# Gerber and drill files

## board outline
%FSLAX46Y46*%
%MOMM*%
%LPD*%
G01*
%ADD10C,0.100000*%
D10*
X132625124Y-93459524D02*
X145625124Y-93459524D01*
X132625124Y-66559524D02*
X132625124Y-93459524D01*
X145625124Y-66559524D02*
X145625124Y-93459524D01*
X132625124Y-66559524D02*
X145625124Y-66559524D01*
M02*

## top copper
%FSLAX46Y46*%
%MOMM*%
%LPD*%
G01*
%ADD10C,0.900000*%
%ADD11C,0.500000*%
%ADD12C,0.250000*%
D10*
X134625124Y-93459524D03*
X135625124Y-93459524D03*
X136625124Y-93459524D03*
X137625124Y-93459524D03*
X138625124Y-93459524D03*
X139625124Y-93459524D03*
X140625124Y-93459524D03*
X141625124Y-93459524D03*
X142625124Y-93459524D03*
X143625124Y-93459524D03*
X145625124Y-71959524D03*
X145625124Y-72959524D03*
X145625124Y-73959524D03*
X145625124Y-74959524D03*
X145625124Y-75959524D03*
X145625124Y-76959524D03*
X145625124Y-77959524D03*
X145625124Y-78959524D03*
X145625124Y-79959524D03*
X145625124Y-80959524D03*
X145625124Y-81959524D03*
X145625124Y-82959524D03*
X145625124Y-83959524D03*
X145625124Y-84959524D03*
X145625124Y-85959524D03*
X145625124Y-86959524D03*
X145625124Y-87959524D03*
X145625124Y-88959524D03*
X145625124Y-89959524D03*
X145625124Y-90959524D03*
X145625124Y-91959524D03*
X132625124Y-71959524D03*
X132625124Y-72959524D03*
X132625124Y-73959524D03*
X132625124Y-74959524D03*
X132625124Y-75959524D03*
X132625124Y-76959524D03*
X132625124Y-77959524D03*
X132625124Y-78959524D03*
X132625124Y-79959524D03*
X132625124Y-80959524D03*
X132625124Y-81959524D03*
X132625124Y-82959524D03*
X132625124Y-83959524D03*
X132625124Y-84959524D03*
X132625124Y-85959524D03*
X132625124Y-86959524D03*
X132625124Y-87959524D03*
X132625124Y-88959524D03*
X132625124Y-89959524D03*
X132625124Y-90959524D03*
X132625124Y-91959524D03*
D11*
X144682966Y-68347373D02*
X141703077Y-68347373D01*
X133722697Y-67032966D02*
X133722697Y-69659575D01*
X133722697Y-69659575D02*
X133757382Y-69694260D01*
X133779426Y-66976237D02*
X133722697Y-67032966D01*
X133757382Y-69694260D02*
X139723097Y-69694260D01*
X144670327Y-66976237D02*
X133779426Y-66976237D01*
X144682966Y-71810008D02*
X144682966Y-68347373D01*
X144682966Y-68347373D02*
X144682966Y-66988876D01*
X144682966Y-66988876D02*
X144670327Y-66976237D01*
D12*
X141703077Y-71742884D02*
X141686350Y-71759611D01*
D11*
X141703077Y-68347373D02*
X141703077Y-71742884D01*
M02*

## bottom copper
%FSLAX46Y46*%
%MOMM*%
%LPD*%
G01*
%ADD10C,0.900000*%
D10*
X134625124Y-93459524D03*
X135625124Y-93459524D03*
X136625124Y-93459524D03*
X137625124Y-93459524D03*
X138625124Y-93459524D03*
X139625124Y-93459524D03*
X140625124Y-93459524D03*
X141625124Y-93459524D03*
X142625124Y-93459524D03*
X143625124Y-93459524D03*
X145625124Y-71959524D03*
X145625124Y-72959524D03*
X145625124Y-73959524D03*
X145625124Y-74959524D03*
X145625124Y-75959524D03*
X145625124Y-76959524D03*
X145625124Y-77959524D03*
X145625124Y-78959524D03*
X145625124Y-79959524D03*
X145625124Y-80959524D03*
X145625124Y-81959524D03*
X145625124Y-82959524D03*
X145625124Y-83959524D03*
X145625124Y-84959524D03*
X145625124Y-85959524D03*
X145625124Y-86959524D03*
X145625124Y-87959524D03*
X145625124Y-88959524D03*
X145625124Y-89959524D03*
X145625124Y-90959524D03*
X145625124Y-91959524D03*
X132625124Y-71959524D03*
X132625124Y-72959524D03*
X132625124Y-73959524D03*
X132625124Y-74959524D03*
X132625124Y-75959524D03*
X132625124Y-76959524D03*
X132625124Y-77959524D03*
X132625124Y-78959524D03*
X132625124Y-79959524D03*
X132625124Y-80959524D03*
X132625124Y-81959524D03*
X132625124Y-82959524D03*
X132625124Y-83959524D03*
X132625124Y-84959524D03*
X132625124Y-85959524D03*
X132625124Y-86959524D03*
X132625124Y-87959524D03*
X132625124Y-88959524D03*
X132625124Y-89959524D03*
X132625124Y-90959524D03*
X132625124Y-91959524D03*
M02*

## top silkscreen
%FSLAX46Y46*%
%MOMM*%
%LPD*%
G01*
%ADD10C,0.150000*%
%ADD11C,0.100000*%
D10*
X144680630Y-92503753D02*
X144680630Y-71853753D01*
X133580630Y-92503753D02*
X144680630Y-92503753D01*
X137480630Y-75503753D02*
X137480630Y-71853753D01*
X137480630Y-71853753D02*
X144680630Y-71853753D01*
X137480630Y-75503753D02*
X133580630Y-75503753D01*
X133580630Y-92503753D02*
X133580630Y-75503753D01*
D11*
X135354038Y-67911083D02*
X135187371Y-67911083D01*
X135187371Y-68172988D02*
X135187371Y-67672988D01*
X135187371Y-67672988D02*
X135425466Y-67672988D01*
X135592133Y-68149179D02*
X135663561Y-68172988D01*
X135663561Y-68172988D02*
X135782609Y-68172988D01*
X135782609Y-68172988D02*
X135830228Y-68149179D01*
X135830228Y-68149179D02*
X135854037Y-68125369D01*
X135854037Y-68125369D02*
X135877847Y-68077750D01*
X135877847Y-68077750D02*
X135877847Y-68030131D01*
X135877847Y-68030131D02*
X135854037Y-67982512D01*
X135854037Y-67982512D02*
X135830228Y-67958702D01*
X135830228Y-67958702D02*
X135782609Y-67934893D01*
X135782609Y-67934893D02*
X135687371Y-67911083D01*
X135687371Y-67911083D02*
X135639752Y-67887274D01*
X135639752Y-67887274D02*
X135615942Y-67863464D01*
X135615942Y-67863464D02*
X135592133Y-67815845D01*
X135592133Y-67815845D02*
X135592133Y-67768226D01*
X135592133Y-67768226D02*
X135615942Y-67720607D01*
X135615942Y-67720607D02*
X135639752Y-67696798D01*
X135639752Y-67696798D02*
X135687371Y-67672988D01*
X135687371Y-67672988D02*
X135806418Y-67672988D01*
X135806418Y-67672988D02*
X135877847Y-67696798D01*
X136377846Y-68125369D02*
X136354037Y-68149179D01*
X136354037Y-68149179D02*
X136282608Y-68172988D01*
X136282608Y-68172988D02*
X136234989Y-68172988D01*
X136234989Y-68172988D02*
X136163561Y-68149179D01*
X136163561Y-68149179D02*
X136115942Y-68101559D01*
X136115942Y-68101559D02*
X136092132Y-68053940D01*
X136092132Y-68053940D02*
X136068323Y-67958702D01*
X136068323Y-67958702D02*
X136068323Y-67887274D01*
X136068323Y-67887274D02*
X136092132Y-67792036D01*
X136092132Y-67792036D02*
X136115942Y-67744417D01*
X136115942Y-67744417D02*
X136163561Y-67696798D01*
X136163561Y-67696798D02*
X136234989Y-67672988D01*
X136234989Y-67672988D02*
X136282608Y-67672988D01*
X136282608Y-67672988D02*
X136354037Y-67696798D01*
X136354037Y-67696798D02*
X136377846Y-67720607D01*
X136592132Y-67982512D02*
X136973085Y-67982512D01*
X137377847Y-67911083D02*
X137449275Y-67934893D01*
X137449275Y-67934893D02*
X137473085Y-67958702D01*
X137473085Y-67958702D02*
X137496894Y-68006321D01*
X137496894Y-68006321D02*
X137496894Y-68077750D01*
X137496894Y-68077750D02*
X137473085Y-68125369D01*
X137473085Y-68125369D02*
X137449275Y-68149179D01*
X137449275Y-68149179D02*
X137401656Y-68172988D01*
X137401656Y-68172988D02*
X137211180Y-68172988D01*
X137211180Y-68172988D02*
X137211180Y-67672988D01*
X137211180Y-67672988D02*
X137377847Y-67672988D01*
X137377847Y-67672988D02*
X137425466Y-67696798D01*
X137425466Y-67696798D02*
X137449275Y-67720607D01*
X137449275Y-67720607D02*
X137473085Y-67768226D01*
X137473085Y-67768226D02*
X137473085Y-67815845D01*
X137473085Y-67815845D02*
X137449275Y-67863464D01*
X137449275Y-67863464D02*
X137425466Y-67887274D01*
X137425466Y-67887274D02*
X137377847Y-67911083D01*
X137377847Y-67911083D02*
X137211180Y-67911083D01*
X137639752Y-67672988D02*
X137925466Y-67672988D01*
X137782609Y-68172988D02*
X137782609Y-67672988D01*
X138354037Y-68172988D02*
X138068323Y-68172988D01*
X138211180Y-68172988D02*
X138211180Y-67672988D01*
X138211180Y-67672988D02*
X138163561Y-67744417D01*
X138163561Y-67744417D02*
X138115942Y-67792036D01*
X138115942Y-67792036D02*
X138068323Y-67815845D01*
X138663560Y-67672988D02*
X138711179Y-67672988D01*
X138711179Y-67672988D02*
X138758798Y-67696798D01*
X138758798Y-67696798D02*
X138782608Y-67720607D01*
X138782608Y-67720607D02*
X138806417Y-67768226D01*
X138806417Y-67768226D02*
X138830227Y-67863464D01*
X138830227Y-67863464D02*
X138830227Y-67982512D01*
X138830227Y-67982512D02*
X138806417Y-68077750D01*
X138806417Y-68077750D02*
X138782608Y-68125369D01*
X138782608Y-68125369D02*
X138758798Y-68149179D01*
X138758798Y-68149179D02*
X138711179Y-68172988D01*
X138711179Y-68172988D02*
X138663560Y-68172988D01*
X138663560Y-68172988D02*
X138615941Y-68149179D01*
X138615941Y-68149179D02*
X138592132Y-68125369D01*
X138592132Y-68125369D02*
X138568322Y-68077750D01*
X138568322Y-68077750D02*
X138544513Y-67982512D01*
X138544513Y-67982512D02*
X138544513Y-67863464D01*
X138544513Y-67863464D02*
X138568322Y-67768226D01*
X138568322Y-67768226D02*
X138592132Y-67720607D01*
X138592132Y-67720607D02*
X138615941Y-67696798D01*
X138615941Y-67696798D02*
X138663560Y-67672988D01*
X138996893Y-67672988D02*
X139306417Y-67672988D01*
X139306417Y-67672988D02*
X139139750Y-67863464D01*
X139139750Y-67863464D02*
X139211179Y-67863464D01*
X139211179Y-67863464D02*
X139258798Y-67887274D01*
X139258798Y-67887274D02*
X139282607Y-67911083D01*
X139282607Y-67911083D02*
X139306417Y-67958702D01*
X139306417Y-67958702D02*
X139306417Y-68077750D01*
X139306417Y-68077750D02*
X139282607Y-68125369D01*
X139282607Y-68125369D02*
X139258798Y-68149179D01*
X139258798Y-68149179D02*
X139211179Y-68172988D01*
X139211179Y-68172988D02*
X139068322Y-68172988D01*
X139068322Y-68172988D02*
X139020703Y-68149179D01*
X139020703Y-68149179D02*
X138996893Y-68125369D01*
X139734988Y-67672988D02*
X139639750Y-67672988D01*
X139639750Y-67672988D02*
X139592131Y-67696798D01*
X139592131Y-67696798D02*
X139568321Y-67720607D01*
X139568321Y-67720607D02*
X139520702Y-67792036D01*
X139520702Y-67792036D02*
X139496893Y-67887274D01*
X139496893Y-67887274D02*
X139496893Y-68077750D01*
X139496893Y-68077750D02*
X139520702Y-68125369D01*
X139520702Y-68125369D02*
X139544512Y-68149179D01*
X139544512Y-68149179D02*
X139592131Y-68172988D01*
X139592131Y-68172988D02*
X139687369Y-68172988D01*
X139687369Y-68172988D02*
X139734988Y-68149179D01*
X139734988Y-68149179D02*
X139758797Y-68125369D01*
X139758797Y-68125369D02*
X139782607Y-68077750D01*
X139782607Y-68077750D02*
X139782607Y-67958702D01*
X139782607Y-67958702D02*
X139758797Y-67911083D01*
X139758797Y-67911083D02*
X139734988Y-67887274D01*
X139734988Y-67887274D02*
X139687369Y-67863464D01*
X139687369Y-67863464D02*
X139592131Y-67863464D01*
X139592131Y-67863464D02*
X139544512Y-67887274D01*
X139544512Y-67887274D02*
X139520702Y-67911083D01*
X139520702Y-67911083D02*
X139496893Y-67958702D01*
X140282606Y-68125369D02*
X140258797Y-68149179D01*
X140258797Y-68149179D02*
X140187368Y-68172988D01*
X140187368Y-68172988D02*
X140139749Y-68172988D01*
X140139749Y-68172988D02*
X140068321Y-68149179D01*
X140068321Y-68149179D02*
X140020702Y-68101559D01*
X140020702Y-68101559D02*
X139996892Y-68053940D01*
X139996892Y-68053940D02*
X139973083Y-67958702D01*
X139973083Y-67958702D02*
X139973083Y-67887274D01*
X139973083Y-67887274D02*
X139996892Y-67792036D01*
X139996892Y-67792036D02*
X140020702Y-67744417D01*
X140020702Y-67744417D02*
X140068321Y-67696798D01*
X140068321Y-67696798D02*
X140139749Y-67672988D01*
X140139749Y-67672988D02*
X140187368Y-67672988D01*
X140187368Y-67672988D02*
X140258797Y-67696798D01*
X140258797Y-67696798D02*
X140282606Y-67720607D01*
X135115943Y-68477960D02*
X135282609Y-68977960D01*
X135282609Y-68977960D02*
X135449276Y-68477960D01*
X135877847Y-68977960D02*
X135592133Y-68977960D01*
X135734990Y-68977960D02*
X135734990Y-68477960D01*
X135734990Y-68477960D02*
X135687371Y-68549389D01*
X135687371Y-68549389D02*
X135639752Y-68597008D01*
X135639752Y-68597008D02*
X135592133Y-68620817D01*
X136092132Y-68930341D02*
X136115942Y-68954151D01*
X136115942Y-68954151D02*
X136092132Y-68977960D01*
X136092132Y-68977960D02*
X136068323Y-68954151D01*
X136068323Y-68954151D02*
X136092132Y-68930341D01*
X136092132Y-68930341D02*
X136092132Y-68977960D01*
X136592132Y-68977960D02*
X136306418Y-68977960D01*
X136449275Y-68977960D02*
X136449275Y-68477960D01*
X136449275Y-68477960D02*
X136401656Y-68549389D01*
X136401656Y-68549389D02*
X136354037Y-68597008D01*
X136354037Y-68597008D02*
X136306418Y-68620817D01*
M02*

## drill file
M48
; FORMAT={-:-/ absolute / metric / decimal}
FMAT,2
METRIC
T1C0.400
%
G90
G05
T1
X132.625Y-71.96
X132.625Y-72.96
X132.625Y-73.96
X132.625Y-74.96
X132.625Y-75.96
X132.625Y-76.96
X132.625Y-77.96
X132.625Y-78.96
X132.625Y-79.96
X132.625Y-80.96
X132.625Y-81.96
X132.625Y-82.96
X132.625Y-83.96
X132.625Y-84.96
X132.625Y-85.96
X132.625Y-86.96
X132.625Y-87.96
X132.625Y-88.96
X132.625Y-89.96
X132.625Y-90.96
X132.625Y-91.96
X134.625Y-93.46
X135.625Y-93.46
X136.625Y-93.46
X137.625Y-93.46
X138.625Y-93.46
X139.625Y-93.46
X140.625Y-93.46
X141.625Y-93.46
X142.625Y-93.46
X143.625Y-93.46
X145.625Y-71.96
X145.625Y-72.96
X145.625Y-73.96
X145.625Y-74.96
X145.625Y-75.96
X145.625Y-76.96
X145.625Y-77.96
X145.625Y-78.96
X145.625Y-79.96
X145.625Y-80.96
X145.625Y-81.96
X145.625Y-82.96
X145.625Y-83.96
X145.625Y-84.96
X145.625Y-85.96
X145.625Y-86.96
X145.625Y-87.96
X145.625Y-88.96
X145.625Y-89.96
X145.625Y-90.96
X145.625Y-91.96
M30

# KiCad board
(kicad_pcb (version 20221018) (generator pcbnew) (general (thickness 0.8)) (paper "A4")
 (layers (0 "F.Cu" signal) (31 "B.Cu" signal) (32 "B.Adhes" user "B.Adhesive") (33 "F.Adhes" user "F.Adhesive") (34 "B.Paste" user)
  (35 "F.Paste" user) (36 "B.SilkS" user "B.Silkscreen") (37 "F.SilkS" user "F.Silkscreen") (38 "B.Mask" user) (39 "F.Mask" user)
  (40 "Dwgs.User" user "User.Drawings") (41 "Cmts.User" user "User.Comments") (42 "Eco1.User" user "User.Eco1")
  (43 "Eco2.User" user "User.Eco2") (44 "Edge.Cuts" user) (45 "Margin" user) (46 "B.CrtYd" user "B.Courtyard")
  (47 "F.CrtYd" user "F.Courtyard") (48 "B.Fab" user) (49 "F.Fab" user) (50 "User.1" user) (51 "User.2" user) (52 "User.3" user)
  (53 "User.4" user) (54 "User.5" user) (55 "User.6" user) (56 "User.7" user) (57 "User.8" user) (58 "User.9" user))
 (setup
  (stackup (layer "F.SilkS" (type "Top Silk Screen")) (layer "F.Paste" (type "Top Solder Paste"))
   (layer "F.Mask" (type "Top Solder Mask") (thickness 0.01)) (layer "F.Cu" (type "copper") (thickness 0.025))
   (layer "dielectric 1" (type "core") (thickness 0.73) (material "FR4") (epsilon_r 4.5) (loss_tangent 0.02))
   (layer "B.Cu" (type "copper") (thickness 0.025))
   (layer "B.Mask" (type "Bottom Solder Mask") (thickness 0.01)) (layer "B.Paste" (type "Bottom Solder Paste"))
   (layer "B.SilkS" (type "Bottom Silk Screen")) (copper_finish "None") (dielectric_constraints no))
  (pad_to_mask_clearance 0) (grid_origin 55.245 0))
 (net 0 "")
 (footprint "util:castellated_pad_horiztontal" (layer "F.Cu") (at 134.625124 93.459524)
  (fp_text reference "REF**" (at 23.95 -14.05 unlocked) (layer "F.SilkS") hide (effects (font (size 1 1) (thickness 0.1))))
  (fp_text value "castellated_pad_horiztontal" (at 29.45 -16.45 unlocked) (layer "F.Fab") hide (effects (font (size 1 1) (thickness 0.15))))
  (pad "1" thru_hole circle (at 0 0) (size 0.9 0.9) (drill 0.4) (layers "*.Cu" "*.Mask"))
  (pad "1" thru_hole circle (at 1 0) (size 0.9 0.9) (drill 0.4) (layers "*.Cu" "*.Mask"))
  (pad "1" thru_hole circle (at 2 0) (size 0.9 0.9) (drill 0.4) (layers "*.Cu" "*.Mask"))
  (pad "1" thru_hole circle (at 3 0) (size 0.9 0.9) (drill 0.4) (layers "*.Cu" "*.Mask"))
  (pad "1" thru_hole circle (at 4 0) (size 0.9 0.9) (drill 0.4) (layers "*.Cu" "*.Mask"))
  (pad "1" thru_hole circle (at 5 0) (size 0.9 0.9) (drill 0.4) (layers "*.Cu" "*.Mask"))
  (pad "1" thru_hole circle (at 6 0) (size 0.9 0.9) (drill 0.4) (layers "*.Cu" "*.Mask"))
  (pad "1" thru_hole circle (at 7 0) (size 0.9 0.9) (drill 0.4) (layers "*.Cu" "*.Mask"))
  (pad "1" thru_hole circle (at 8 0) (size 0.9 0.9) (drill 0.4) (layers "*.Cu" "*.Mask"))
  (pad "1" thru_hole circle (at 9 0) (size 0.9 0.9) (drill 0.4) (layers "*.Cu" "*.Mask")))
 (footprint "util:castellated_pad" (layer "F.Cu") (at 145.625124 71.959524)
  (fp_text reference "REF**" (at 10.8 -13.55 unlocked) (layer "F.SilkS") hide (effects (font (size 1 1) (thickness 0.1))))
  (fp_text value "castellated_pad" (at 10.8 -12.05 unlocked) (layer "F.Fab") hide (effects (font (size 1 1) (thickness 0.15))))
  (pad "1" thru_hole circle (at 0 0) (size 0.9 0.9) (drill 0.4) (layers "*.Cu" "*.Mask"))
  (pad "1" thru_hole circle (at 0 1) (size 0.9 0.9) (drill 0.4) (layers "*.Cu" "*.Mask"))
  (pad "1" thru_hole circle (at 0 2) (size 0.9 0.9) (drill 0.4) (layers "*.Cu" "*.Mask"))
  (pad "1" thru_hole circle (at 0 3) (size 0.9 0.9) (drill 0.4) (layers "*.Cu" "*.Mask"))
  (pad "1" thru_hole circle (at 0 4) (size 0.9 0.9) (drill 0.4) (layers "*.Cu" "*.Mask"))
  (pad "1" thru_hole circle (at 0 5) (size 0.9 0.9) (drill 0.4) (layers "*.Cu" "*.Mask"))
  (pad "1" thru_hole circle (at 0 6) (size 0.9 0.9) (drill 0.4) (layers "*.Cu" "*.Mask"))
  (pad "1" thru_hole circle (at 0 7) (size 0.9 0.9) (drill 0.4) (layers "*.Cu" "*.Mask"))
  (pad "1" thru_hole circle (at 0 8) (size 0.9 0.9) (drill 0.4) (layers "*.Cu" "*.Mask"))
  (pad "1" thru_hole circle (at 0 9) (size 0.9 0.9) (drill 0.4) (layers "*.Cu" "*.Mask"))
  (pad "1" thru_hole circle (at 0 10) (size 0.9 0.9) (drill 0.4) (layers "*.Cu" "*.Mask"))
  (pad "1" thru_hole circle (at 0 11) (size 0.9 0.9) (drill 0.4) (layers "*.Cu" "*.Mask"))
  (pad "1" thru_hole circle (at 0 12) (size 0.9 0.9) (drill 0.4) (layers "*.Cu" "*.Mask"))
  (pad "1" thru_hole circle (at 0 13) (size 0.9 0.9) (drill 0.4) (layers "*.Cu" "*.Mask"))
  (pad "1" thru_hole circle (at 0 14) (size 0.9 0.9) (drill 0.4) (layers "*.Cu" "*.Mask"))
  (pad "1" thru_hole circle (at 0 15) (size 0.9 0.9) (drill 0.4) (layers "*.Cu" "*.Mask"))
  (pad "1" thru_hole circle (at 0 16) (size 0.9 0.9) (drill 0.4) (layers "*.Cu" "*.Mask"))
  (pad "1" thru_hole circle (at 0 17) (size 0.9 0.9) (drill 0.4) (layers "*.Cu" "*.Mask"))
  (pad "1" thru_hole circle (at 0 18) (size 0.9 0.9) (drill 0.4) (layers "*.Cu" "*.Mask"))
  (pad "1" thru_hole circle (at 0 19) (size 0.9 0.9) (drill 0.4) (layers "*.Cu" "*.Mask"))
  (pad "1" thru_hole circle (at 0 20) (size 0.9 0.9) (drill 0.4) (layers "*.Cu" "*.Mask")))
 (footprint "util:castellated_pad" (layer "F.Cu") (at 132.625124 71.959524)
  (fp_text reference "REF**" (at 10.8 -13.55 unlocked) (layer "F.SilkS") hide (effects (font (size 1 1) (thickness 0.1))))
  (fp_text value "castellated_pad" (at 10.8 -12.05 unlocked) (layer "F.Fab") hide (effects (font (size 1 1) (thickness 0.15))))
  (pad "1" thru_hole circle (at 0 0) (size 0.9 0.9) (drill 0.4) (layers "*.Cu" "*.Mask"))
  (pad "1" thru_hole circle (at 0 1) (size 0.9 0.9) (drill 0.4) (layers "*.Cu" "*.Mask"))
  (pad "1" thru_hole circle (at 0 2) (size 0.9 0.9) (drill 0.4) (layers "*.Cu" "*.Mask"))
  (pad "1" thru_hole circle (at 0 3) (size 0.9 0.9) (drill 0.4) (layers "*.Cu" "*.Mask"))
  (pad "1" thru_hole circle (at 0 4) (size 0.9 0.9) (drill 0.4) (layers "*.Cu" "*.Mask"))
  (pad "1" thru_hole circle (at 0 5) (size 0.9 0.9) (drill 0.4) (layers "*.Cu" "*.Mask"))
  (pad "1" thru_hole circle (at 0 6) (size 0.9 0.9) (drill 0.4) (layers "*.Cu" "*.Mask"))
  (pad "1" thru_hole circle (at 0 7) (size 0.9 0.9) (drill 0.4) (layers "*.Cu" "*.Mask"))
  (pad "1" thru_hole circle (at 0 8) (size 0.9 0.9) (drill 0.4) (layers "*.Cu" "*.Mask"))
  (pad "1" thru_hole circle (at 0 9) (size 0.9 0.9) (drill 0.4) (layers "*.Cu" "*.Mask"))
  (pad "1" thru_hole circle (at 0 10) (size 0.9 0.9) (drill 0.4) (layers "*.Cu" "*.Mask"))
  (pad "1" thru_hole circle (at 0 11) (size 0.9 0.9) (drill 0.4) (layers "*.Cu" "*.Mask"))
  (pad "1" thru_hole circle (at 0 12) (size 0.9 0.9) (drill 0.4) (layers "*.Cu" "*.Mask"))
  (pad "1" thru_hole circle (at 0 13) (size 0.9 0.9) (drill 0.4) (layers "*.Cu" "*.Mask"))
  (pad "1" thru_hole circle (at 0 14) (size 0.9 0.9) (drill 0.4) (layers "*.Cu" "*.Mask"))
  (pad "1" thru_hole circle (at 0 15) (size 0.9 0.9) (drill 0.4) (layers "*.Cu" "*.Mask"))
  (pad "1" thru_hole circle (at 0 16) (size 0.9 0.9) (drill 0.4) (layers "*.Cu" "*.Mask"))
  (pad "1" thru_hole circle (at 0 17) (size 0.9 0.9) (drill 0.4) (layers "*.Cu" "*.Mask"))
  (pad "1" thru_hole circle (at 0 18) (size 0.9 0.9) (drill 0.4) (layers "*.Cu" "*.Mask"))
  (pad "1" thru_hole circle (at 0 19) (size 0.9 0.9) (drill 0.4) (layers "*.Cu" "*.Mask"))
  (pad "1" thru_hole circle (at 0 20) (size 0.9 0.9) (drill 0.4) (layers "*.Cu" "*.Mask")))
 (gr_line (start 144.68063 92.503753) (end 144.68063 71.853753) (stroke (width 0.15) (type default)) (layer "F.SilkS"))
 (gr_line (start 133.58063 92.503753) (end 144.68063 92.503753) (stroke (width 0.15) (type default)) (layer "F.SilkS"))
 (gr_line (start 137.48063 75.503753) (end 137.48063 71.853753) (stroke (width 0.15) (type default)) (layer "F.SilkS"))
 (gr_line (start 137.48063 71.853753) (end 144.68063 71.853753) (stroke (width 0.15) (type default)) (layer "F.SilkS"))
 (gr_line (start 137.48063 75.503753) (end 133.58063 75.503753) (stroke (width 0.15) (type default)) (layer "F.SilkS"))
 (gr_line (start 133.58063 92.503753) (end 133.58063 75.503753) (stroke (width 0.15) (type default)) (layer "F.SilkS"))
 (gr_line (start 132.625124 93.459524) (end 145.625124 93.459524) (stroke (width 0.1) (type default)) (layer "Edge.Cuts"))
 (gr_line (start 132.625124 66.559524) (end 132.625124 93.459524) (stroke (width 0.1) (type default)) (layer "Edge.Cuts"))
 (gr_line (start 145.625124 66.559524) (end 145.625124 93.459524) (stroke (width 0.1) (type default)) (layer "Edge.Cuts"))
 (gr_line (start 132.625124 66.559524) (end 145.625124 66.559524) (stroke (width 0.1) (type default)) (layer "Edge.Cuts"))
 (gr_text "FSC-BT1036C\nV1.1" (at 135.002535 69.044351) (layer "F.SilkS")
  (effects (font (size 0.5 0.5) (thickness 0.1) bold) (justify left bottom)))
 (segment (start 144.682966 68.347373) (end 141.703077 68.347373) (width 0.5) (layer "F.Cu") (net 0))
 (segment (start 133.722697 67.032966) (end 133.722697 69.659575) (width 0.5) (layer "F.Cu") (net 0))
 (segment (start 133.722697 69.659575) (end 133.757382 69.69426) (width 0.5) (layer "F.Cu") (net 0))
 (segment (start 133.779426 66.976237) (end 133.722697 67.032966) (width 0.5) (layer "F.Cu") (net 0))
 (segment (start 133.757382 69.69426) (end 139.723097 69.69426) (width 0.5) (layer "F.Cu") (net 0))
 (segment (start 144.670327 66.976237) (end 133.779426 66.976237) (width 0.5) (layer "F.Cu") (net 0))
 (segment (start 144.682966 71.810008) (end 144.682966 68.347373) (width 0.5) (layer "F.Cu") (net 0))
 (segment (start 144.682966 68.347373) (end 144.682966 66.988876) (width 0.5) (layer "F.Cu") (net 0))
 (segment (start 144.682966 66.988876) (end 144.670327 66.976237) (width 0.5) (layer "F.Cu") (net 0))
 (segment (start 141.703077 71.742884) (end 141.68635 71.759611) (width 0.25) (layer "F.Cu") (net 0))
 (segment (start 141.703077 68.347373) (end 141.703077 71.742884) (width 0.5) (layer "F.Cu") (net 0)))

